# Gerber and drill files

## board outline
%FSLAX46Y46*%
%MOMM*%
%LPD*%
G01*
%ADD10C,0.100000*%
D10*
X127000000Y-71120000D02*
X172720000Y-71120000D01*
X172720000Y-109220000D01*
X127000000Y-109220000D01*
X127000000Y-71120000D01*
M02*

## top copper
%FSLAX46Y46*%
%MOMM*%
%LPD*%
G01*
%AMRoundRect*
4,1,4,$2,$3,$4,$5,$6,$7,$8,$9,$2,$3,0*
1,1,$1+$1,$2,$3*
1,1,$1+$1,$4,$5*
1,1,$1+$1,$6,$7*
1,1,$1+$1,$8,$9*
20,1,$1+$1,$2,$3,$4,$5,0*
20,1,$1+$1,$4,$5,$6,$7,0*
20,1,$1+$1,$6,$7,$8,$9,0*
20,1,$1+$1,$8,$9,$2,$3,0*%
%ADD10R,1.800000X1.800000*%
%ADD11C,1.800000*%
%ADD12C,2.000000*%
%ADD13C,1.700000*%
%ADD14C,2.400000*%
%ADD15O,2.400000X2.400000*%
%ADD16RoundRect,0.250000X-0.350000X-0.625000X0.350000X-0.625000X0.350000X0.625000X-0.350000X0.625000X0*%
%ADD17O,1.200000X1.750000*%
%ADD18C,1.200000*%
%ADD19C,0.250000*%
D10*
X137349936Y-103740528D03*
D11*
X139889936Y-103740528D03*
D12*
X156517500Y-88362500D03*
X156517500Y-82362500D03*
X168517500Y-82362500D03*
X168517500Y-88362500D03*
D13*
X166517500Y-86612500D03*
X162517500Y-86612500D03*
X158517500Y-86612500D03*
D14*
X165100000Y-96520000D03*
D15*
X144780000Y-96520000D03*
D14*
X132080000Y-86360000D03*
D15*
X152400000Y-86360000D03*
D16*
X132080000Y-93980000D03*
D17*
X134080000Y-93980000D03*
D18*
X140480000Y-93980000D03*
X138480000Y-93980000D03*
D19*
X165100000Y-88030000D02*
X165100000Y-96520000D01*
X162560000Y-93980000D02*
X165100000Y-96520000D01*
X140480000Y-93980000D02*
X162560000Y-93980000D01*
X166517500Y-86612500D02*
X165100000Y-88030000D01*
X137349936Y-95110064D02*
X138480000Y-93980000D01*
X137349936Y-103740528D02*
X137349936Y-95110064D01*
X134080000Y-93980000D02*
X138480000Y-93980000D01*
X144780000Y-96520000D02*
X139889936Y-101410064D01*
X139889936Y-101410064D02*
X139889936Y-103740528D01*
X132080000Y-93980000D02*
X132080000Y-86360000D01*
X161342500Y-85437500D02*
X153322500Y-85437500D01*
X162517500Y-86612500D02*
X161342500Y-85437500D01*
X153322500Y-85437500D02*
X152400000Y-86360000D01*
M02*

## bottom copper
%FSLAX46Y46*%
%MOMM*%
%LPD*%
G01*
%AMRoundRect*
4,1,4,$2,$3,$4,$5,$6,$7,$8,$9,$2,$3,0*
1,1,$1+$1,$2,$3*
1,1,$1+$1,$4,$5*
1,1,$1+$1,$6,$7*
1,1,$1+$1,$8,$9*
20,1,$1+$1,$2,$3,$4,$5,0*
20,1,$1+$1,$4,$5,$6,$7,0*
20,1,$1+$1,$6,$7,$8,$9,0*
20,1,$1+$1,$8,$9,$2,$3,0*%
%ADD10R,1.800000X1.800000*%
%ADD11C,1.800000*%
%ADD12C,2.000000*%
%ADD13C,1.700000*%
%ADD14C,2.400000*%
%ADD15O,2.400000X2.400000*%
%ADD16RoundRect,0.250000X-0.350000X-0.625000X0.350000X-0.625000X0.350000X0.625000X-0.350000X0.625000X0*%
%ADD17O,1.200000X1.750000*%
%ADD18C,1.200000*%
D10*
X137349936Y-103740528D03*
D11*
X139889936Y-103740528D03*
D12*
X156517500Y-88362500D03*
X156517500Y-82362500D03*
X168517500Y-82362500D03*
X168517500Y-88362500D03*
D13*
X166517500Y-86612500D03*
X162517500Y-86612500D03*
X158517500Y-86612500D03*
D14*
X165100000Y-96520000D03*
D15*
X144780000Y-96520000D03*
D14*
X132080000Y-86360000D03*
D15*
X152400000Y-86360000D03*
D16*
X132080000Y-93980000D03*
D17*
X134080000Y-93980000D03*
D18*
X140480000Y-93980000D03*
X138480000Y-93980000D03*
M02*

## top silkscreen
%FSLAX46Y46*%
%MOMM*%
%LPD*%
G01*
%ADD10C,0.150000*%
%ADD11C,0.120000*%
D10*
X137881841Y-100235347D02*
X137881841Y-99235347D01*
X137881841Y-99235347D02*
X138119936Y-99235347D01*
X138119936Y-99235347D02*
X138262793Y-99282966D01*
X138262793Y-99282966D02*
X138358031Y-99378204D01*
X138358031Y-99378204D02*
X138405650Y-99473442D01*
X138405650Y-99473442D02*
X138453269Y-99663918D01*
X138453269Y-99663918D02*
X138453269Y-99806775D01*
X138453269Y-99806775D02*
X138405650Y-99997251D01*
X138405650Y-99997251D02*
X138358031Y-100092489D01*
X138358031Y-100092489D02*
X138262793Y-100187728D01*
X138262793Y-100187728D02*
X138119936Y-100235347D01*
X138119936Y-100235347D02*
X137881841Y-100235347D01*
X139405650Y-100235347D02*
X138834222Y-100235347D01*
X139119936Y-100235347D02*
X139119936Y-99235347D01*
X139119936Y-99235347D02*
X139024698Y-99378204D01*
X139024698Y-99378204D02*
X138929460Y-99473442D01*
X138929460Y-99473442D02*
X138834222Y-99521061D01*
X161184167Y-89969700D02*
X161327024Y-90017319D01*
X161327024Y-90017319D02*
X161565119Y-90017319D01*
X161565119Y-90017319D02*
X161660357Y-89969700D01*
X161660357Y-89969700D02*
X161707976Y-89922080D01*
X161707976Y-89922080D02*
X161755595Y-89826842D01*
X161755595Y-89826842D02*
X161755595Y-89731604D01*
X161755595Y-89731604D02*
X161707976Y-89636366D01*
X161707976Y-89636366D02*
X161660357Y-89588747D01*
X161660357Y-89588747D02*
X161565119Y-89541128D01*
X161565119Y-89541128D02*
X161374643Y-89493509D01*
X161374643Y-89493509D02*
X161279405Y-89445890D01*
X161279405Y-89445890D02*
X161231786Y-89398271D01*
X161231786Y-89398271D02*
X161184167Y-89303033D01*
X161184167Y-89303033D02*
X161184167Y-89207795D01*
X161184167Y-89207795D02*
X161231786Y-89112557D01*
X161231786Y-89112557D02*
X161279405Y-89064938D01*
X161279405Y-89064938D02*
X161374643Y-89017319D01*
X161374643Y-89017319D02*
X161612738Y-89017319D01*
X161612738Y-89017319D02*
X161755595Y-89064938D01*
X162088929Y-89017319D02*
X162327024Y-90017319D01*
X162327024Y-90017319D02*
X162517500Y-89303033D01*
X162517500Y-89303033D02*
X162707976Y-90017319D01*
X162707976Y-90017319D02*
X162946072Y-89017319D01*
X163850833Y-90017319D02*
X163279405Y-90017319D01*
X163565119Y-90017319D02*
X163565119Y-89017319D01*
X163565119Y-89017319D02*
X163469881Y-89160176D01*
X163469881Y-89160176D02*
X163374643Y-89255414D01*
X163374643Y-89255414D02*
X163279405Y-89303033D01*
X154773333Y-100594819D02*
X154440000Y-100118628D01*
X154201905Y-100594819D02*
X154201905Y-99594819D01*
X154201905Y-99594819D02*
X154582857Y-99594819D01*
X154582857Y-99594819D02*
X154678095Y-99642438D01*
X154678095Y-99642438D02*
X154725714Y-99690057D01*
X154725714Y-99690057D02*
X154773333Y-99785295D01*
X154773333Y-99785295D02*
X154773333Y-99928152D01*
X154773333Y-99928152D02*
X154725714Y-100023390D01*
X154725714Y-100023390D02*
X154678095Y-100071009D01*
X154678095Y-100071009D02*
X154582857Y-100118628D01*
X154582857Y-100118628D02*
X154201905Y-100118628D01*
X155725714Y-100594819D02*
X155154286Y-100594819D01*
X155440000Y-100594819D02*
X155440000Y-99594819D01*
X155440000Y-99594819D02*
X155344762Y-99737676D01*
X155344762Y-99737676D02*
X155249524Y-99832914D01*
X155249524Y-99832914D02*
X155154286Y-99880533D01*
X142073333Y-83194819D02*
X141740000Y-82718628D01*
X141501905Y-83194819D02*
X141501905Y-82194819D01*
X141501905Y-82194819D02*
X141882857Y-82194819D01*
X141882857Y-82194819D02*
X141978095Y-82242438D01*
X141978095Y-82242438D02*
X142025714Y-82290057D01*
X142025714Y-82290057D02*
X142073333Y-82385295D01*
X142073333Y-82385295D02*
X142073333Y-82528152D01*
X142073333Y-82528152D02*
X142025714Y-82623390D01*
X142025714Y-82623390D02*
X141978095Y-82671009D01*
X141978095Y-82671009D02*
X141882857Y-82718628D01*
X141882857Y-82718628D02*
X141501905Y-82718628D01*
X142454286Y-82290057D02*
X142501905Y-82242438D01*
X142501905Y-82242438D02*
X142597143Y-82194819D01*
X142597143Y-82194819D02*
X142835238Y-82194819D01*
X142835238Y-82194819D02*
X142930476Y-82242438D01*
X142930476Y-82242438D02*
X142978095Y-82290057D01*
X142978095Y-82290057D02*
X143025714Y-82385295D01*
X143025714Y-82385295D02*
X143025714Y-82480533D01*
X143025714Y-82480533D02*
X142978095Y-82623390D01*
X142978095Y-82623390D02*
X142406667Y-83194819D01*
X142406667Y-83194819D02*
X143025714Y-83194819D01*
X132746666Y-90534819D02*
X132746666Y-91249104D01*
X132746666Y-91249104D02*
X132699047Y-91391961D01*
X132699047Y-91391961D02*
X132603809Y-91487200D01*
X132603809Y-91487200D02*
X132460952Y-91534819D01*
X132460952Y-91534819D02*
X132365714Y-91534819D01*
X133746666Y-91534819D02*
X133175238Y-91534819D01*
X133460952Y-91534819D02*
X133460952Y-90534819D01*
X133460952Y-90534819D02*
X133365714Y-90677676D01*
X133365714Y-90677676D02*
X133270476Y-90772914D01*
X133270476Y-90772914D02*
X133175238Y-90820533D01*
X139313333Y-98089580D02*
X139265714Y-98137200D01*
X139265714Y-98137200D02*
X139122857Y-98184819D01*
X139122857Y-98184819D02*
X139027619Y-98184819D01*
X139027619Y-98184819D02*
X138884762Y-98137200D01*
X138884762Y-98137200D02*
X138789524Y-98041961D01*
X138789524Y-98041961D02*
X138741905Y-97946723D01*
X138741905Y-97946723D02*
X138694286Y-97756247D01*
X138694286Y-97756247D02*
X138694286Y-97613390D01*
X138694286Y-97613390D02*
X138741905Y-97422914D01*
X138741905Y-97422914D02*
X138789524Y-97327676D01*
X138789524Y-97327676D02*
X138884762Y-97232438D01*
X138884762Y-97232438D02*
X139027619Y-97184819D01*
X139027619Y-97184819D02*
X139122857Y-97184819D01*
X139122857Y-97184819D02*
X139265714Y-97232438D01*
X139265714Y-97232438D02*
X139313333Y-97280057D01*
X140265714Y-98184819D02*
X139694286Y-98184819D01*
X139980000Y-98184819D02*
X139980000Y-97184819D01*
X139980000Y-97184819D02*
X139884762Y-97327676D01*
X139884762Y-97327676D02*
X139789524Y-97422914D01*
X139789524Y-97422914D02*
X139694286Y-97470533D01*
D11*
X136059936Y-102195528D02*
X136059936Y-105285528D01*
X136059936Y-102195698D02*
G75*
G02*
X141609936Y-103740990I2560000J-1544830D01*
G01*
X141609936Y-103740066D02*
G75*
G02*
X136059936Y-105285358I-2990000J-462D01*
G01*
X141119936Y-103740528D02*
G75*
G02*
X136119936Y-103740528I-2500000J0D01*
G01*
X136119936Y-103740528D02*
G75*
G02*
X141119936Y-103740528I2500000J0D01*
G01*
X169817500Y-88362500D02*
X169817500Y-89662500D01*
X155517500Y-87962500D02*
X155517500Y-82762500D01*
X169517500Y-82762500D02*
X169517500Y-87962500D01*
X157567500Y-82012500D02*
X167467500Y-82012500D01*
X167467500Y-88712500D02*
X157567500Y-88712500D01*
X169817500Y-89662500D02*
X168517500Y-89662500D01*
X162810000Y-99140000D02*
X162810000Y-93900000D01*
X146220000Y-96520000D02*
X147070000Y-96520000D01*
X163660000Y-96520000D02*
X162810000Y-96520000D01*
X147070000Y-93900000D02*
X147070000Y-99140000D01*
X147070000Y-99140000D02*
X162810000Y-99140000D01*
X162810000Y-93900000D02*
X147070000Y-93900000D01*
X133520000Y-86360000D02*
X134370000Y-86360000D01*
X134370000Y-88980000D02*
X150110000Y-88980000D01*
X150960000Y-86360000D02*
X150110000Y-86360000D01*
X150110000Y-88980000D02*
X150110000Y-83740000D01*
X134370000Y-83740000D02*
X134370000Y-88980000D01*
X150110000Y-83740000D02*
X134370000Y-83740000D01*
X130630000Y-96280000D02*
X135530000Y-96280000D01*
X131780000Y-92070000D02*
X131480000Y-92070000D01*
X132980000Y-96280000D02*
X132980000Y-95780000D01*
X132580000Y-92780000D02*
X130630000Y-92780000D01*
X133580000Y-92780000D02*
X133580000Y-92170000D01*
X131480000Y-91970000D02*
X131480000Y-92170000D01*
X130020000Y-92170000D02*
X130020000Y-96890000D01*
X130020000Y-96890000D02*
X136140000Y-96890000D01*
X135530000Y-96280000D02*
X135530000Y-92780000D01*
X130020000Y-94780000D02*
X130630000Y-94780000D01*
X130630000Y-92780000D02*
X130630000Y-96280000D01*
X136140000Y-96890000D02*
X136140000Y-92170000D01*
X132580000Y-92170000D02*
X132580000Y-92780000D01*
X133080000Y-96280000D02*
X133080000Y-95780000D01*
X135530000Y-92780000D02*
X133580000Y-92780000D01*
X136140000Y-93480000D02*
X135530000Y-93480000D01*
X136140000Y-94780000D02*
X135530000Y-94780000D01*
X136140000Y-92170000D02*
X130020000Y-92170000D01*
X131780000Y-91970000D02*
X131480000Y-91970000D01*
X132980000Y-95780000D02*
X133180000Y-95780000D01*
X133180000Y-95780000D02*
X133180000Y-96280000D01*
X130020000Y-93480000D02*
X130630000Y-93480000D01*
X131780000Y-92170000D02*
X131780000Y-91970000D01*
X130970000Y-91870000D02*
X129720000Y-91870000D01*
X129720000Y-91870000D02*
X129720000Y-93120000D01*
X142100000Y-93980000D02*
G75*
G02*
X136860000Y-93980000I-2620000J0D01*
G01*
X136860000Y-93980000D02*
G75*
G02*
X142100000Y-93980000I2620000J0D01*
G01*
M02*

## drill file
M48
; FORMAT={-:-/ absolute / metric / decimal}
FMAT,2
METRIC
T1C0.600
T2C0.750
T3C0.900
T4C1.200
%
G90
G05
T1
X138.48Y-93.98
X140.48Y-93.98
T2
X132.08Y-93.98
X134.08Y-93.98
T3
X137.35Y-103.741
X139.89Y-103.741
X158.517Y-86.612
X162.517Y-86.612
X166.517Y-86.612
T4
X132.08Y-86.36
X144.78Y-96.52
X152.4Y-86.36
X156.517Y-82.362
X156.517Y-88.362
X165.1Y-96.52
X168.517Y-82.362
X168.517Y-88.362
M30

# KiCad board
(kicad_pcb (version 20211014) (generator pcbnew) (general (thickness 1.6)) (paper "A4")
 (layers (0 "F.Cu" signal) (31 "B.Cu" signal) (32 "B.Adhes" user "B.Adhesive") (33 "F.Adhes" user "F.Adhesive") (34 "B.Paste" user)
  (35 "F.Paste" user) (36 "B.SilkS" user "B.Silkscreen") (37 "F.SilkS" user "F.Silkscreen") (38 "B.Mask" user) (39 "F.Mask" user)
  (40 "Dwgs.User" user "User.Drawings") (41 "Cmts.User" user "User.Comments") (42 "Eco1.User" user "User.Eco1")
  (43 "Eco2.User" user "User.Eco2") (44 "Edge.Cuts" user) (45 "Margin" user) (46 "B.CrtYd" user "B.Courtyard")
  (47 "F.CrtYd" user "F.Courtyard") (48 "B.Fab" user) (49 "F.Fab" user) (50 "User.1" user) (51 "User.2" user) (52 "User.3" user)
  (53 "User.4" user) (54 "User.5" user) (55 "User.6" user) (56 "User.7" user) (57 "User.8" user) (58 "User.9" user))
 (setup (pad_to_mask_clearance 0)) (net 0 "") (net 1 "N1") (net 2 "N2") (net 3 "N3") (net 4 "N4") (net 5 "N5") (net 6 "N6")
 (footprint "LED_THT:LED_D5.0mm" (layer "F.Cu") (at 137.349936 103.740528)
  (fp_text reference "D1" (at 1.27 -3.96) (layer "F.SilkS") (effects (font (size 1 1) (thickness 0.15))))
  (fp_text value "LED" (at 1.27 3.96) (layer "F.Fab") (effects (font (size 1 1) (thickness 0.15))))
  (fp_line (start -1.29 -1.545) (end -1.29 1.545) (layer "F.SilkS") (width 0.12))
  (fp_arc (start -1.29 -1.54483) (mid 2.072002 -2.880433) (end 4.26 0.000462) (layer "F.SilkS") (width 0.12))
  (fp_arc (start 4.26 -0.000462) (mid 2.072002 2.880433) (end -1.29 1.54483) (layer "F.SilkS") (width 0.12))
  (fp_circle (center 1.27 0) (end 3.77 0) (layer "F.SilkS") (width 0.12) (fill none))
  (pad "1" thru_hole rect (at 0 0) (size 1.8 1.8) (drill 0.9) (layers *.Cu *.Mask) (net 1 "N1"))
  (pad "2" thru_hole circle (at 2.54 0) (size 1.8 1.8) (drill 0.9) (layers *.Cu *.Mask) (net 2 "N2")))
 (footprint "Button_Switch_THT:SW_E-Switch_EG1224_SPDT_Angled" (layer "F.Cu") (at 166.5175 86.6125 180)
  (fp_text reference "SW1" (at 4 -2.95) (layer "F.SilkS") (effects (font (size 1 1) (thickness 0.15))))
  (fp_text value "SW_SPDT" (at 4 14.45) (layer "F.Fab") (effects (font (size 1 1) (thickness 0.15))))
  (fp_line (start -3.3 -1.75) (end -3.3 -3.05) (layer "F.SilkS") (width 0.12))
  (fp_line (start 11 -1.35) (end 11 3.85) (layer "F.SilkS") (width 0.12))
  (fp_line (start -3 3.85) (end -3 -1.35) (layer "F.SilkS") (width 0.12))
  (fp_line (start 8.95 4.6) (end -0.95 4.6) (layer "F.SilkS") (width 0.12))
  (fp_line (start -0.95 -2.1) (end 8.95 -2.1) (layer "F.SilkS") (width 0.12))
  (fp_line (start -3.3 -3.05) (end -2 -3.05) (layer "F.SilkS") (width 0.12))
  (pad "" thru_hole circle (at 10 -1.75 180) (size 2 2) (drill 1.2) (layers *.Cu *.Mask))
  (pad "" thru_hole circle (at 10 4.25 180) (size 2 2) (drill 1.2) (layers *.Cu *.Mask))
  (pad "" thru_hole circle (at -2 4.25 180) (size 2 2) (drill 1.2) (layers *.Cu *.Mask))
  (pad "" thru_hole circle (at -2 -1.75 180) (size 2 2) (drill 1.2) (layers *.Cu *.Mask))
  (pad "1" thru_hole circle (at 0 0 180) (size 1.7 1.7) (drill 0.9) (layers *.Cu *.Mask) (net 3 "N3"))
  (pad "2" thru_hole circle (at 4 0 180) (size 1.7 1.7) (drill 0.9) (layers *.Cu *.Mask) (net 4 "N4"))
  (pad "3" thru_hole circle (at 8 0 180) (size 1.7 1.7) (drill 0.9) (layers *.Cu *.Mask) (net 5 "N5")))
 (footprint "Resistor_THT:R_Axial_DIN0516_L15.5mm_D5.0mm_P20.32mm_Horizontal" (layer "F.Cu") (at 165.1 96.52 180)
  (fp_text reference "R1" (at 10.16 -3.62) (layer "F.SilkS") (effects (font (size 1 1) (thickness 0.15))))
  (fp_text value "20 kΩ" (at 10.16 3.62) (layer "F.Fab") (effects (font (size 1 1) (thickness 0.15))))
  (fp_line (start 2.29 -2.62) (end 2.29 2.62) (layer "F.SilkS") (width 0.12))
  (fp_line (start 18.88 0) (end 18.03 0) (layer "F.SilkS") (width 0.12))
  (fp_line (start 1.44 0) (end 2.29 0) (layer "F.SilkS") (width 0.12))
  (fp_line (start 18.03 2.62) (end 18.03 -2.62) (layer "F.SilkS") (width 0.12))
  (fp_line (start 18.03 -2.62) (end 2.29 -2.62) (layer "F.SilkS") (width 0.12))
  (fp_line (start 2.29 2.62) (end 18.03 2.62) (layer "F.SilkS") (width 0.12))
  (pad "1" thru_hole circle (at 0 0 180) (size 2.4 2.4) (drill 1.2) (layers *.Cu *.Mask) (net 3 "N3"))
  (pad "2" thru_hole oval (at 20.32 0 180) (size 2.4 2.4) (drill 1.2) (layers *.Cu *.Mask) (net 2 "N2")))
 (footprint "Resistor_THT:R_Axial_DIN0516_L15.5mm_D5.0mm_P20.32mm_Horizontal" (layer "F.Cu") (at 132.08 86.36)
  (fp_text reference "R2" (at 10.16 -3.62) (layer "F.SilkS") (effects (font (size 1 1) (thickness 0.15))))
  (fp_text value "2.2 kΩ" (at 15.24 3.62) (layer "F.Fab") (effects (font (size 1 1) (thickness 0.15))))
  (fp_line (start 1.44 0) (end 2.29 0) (layer "F.SilkS") (width 0.12))
  (fp_line (start 2.29 2.62) (end 18.03 2.62) (layer "F.SilkS") (width 0.12))
  (fp_line (start 18.88 0) (end 18.03 0) (layer "F.SilkS") (width 0.12))
  (fp_line (start 18.03 2.62) (end 18.03 -2.62) (layer "F.SilkS") (width 0.12))
  (fp_line (start 2.29 -2.62) (end 2.29 2.62) (layer "F.SilkS") (width 0.12))
  (fp_line (start 18.03 -2.62) (end 2.29 -2.62) (layer "F.SilkS") (width 0.12))
  (pad "1" thru_hole circle (at 0 0) (size 2.4 2.4) (drill 1.2) (layers *.Cu *.Mask) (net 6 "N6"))
  (pad "2" thru_hole oval (at 20.32 0) (size 2.4 2.4) (drill 1.2) (layers *.Cu *.Mask) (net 4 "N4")))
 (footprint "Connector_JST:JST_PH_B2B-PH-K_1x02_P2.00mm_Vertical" (layer "F.Cu") (at 132.08 93.98)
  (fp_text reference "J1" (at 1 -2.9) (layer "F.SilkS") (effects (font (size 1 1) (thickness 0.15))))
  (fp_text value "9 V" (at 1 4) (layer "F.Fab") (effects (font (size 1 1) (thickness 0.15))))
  (fp_line (start -1.45 2.3) (end 3.45 2.3) (layer "F.SilkS") (width 0.12))
  (fp_line (start -0.3 -1.91) (end -0.6 -1.91) (layer "F.SilkS") (width 0.12))
  (fp_line (start 0.9 2.3) (end 0.9 1.8) (layer "F.SilkS") (width 0.12))
  (fp_line (start 0.5 -1.2) (end -1.45 -1.2) (layer "F.SilkS") (width 0.12))
  (fp_line (start 1.5 -1.2) (end 1.5 -1.81) (layer "F.SilkS") (width 0.12))
  (fp_line (start -0.6 -2.01) (end -0.6 -1.81) (layer "F.SilkS") (width 0.12))
  (fp_line (start -2.06 -1.81) (end -2.06 2.91) (layer "F.SilkS") (width 0.12))
  (fp_line (start -2.06 2.91) (end 4.06 2.91) (layer "F.SilkS") (width 0.12))
  (fp_line (start 3.45 2.3) (end 3.45 -1.2) (layer "F.SilkS") (width 0.12))
  (fp_line (start -2.06 0.8) (end -1.45 0.8) (layer "F.SilkS") (width 0.12))
  (fp_line (start -1.45 -1.2) (end -1.45 2.3) (layer "F.SilkS") (width 0.12))
  (fp_line (start 4.06 2.91) (end 4.06 -1.81) (layer "F.SilkS") (width 0.12))
  (fp_line (start 0.5 -1.81) (end 0.5 -1.2) (layer "F.SilkS") (width 0.12))
  (fp_line (start 1 2.3) (end 1 1.8) (layer "F.SilkS") (width 0.12))
  (fp_line (start 3.45 -1.2) (end 1.5 -1.2) (layer "F.SilkS") (width 0.12))
  (fp_line (start 4.06 -0.5) (end 3.45 -0.5) (layer "F.SilkS") (width 0.12))
  (fp_line (start 4.06 0.8) (end 3.45 0.8) (layer "F.SilkS") (width 0.12))
  (fp_line (start 4.06 -1.81) (end -2.06 -1.81) (layer "F.SilkS") (width 0.12))
  (fp_line (start -0.3 -2.01) (end -0.6 -2.01) (layer "F.SilkS") (width 0.12))
  (fp_line (start 0.9 1.8) (end 1.1 1.8) (layer "F.SilkS") (width 0.12))
  (fp_line (start 1.1 1.8) (end 1.1 2.3) (layer "F.SilkS") (width 0.12))
  (fp_line (start -2.06 -0.5) (end -1.45 -0.5) (layer "F.SilkS") (width 0.12))
  (fp_line (start -0.3 -1.81) (end -0.3 -2.01) (layer "F.SilkS") (width 0.12))
  (fp_line (start -1.11 -2.11) (end -2.36 -2.11) (layer "F.SilkS") (width 0.12))
  (fp_line (start -2.36 -2.11) (end -2.36 -0.86) (layer "F.SilkS") (width 0.12))
  (pad "1" thru_hole roundrect (at 0 0) (size 1.2 1.75) (drill 0.75) (layers *.Cu *.Mask) (roundrect_rratio 0.208333) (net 6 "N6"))
  (pad "2" thru_hole oval (at 2 0) (size 1.2 1.75) (drill 0.75) (layers *.Cu *.Mask) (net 1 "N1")))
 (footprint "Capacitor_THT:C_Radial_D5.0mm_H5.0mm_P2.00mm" (layer "F.Cu") (at 140.48 93.98 180)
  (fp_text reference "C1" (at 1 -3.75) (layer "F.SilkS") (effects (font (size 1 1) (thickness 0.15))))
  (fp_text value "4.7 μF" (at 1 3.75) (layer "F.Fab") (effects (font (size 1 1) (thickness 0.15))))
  (fp_circle (center 1 0) (end 3.62 0) (layer "F.SilkS") (width 0.12) (fill none))
  (pad "1" thru_hole circle (at 0 0 180) (size 1.2 1.2) (drill 0.6) (layers *.Cu *.Mask) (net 3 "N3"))
  (pad "2" thru_hole circle (at 2 0 180) (size 1.2 1.2) (drill 0.6) (layers *.Cu *.Mask) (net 1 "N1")))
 (gr_rect (start 172.72 109.22) (end 127 71.12) (layer "Edge.Cuts") (width 0.1) (fill none))
 (segment (start 165.1 88.03) (end 165.1 96.52) (width 0.25) (layer "F.Cu") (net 3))
 (segment (start 162.56 93.98) (end 165.1 96.52) (width 0.25) (layer "F.Cu") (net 3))
 (segment (start 140.48 93.98) (end 162.56 93.98) (width 0.25) (layer "F.Cu") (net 3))
 (segment (start 166.5175 86.6125) (end 165.1 88.03) (width 0.25) (layer "F.Cu") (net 3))
 (segment (start 137.349936 95.110064) (end 138.48 93.98) (width 0.25) (layer "F.Cu") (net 1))
 (segment (start 137.349936 103.740528) (end 137.349936 95.110064) (width 0.25) (layer "F.Cu") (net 1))
 (segment (start 134.08 93.98) (end 138.48 93.98) (width 0.25) (layer "F.Cu") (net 1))
 (segment (start 144.78 96.52) (end 139.889936 101.410064) (width 0.25) (layer "F.Cu") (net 2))
 (segment (start 139.889936 101.410064) (end 139.889936 103.740528) (width 0.25) (layer "F.Cu") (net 2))
 (segment (start 132.08 93.98) (end 132.08 86.36) (width 0.25) (layer "F.Cu") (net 6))
 (segment (start 161.3425 85.4375) (end 153.3225 85.4375) (width 0.25) (layer "F.Cu") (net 4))
 (segment (start 162.5175 86.6125) (end 161.3425 85.4375) (width 0.25) (layer "F.Cu") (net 4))
 (segment (start 153.3225 85.4375) (end 152.4 86.36) (width 0.25) (layer "F.Cu") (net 4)))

